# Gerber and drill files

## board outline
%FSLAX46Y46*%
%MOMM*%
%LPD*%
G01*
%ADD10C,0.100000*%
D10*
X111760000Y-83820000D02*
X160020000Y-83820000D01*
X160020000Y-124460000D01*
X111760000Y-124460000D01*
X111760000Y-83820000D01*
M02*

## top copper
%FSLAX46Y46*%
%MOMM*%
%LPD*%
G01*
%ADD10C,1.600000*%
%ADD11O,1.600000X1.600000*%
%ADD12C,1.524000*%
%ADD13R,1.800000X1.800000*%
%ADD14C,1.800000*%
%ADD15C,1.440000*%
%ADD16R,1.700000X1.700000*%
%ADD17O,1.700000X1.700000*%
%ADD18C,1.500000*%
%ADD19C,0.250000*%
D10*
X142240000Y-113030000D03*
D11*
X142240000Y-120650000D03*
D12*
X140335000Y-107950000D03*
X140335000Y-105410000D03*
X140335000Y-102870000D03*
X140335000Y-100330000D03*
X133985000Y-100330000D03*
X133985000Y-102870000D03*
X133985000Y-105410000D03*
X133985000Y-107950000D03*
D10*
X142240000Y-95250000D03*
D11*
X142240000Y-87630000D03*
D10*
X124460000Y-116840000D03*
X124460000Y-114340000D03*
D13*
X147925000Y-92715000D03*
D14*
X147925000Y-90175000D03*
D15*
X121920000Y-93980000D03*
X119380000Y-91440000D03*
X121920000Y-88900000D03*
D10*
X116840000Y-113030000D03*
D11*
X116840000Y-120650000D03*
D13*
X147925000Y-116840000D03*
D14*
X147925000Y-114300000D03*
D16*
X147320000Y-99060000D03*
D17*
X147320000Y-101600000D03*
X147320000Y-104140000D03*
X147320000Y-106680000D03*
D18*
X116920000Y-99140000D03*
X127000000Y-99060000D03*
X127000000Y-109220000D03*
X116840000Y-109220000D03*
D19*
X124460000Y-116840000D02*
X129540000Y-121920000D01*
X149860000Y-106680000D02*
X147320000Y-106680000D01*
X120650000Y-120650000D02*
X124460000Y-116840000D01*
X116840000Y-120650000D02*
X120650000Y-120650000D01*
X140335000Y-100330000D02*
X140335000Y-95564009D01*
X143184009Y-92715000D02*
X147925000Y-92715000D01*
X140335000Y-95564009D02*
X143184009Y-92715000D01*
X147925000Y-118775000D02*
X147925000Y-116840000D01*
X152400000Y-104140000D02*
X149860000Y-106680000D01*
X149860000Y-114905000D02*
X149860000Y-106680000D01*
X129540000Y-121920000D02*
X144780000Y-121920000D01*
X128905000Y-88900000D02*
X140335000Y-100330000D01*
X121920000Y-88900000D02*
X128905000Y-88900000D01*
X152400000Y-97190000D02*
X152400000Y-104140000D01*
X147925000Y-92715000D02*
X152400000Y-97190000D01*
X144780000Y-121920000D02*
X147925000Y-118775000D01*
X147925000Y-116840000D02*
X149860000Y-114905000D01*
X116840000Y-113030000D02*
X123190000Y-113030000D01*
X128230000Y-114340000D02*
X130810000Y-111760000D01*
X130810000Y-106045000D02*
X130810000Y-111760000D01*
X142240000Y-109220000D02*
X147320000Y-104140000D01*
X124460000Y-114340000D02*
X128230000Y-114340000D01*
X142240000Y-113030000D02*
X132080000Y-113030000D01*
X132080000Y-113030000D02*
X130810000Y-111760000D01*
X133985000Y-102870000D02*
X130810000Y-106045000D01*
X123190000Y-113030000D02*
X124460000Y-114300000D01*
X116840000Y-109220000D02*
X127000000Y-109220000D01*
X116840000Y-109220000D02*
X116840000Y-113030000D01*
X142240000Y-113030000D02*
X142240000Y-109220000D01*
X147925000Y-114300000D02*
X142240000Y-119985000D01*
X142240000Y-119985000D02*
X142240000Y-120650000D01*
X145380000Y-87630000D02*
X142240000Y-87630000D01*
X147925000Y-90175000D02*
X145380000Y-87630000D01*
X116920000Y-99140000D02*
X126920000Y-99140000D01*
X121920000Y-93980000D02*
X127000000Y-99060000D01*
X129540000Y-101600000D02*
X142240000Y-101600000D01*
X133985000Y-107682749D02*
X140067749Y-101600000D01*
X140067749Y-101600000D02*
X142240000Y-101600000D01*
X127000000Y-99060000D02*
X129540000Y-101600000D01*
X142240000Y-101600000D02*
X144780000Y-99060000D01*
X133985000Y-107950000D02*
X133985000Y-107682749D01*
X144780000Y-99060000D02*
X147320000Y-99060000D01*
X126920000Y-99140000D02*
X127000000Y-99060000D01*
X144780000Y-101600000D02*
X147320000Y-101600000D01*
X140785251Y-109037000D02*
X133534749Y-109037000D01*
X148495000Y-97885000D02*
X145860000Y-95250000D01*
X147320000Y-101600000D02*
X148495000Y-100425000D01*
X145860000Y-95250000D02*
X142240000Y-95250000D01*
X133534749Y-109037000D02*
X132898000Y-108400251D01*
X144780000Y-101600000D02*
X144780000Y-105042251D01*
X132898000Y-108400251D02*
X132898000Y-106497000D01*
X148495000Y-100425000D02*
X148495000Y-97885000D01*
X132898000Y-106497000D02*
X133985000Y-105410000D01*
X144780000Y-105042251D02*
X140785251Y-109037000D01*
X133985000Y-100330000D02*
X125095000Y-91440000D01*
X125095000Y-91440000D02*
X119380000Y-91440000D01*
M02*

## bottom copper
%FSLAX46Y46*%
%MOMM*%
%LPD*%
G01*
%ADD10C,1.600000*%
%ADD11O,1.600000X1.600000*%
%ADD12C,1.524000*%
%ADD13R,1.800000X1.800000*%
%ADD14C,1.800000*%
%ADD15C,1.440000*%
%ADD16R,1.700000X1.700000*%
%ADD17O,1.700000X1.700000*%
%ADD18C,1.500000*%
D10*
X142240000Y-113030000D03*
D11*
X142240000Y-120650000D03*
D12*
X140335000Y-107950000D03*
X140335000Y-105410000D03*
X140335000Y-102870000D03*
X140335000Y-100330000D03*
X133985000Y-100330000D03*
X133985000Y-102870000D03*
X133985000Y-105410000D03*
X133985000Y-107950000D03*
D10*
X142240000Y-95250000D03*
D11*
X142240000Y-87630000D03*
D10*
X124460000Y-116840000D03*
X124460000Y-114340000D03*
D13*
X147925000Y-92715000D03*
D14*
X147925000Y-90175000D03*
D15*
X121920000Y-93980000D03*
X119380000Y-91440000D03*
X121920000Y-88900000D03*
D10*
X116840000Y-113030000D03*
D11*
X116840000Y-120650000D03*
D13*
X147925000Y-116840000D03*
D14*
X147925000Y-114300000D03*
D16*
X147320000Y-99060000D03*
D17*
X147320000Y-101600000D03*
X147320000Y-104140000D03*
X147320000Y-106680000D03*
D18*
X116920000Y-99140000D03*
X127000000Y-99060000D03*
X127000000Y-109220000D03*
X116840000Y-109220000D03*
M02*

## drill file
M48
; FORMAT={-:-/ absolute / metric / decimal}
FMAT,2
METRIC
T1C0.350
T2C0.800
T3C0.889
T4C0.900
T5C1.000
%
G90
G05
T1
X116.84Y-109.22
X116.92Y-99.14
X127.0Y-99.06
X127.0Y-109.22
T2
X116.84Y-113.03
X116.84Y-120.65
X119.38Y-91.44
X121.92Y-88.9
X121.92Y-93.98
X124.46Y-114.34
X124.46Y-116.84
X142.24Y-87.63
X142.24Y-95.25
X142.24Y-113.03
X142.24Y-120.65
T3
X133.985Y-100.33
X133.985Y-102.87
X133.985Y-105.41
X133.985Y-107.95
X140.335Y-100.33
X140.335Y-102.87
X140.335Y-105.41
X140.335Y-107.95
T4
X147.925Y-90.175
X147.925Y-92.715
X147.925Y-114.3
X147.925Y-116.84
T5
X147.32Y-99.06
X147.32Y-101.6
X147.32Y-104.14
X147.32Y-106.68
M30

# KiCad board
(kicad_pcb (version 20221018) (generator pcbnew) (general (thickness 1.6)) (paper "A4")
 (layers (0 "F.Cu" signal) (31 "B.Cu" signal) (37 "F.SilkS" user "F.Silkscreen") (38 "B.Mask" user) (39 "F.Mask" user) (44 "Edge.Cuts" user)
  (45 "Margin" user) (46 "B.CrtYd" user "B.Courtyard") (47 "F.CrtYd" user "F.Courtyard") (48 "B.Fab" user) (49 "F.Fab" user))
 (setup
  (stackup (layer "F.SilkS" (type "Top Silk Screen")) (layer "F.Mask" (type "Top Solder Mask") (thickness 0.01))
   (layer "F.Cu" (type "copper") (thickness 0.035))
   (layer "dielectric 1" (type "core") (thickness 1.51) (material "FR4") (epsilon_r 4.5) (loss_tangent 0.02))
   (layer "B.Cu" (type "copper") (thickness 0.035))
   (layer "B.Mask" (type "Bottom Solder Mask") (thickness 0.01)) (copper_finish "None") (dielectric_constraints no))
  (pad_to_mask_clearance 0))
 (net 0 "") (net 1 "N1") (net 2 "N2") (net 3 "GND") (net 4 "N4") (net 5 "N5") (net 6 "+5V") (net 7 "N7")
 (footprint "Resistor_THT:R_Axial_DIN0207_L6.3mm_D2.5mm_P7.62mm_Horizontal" (layer "F.Cu") (at 142.24 113.03 -90)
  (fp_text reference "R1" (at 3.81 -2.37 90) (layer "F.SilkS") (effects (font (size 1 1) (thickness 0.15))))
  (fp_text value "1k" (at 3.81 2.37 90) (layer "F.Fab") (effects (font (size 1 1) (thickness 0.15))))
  (pad "1" thru_hole circle (at 0 0 270) (size 1.6 1.6) (drill 0.8) (layers "*.Cu" "*.Mask") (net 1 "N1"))
  (pad "2" thru_hole oval (at 7.62 0 270) (size 1.6 1.6) (drill 0.8) (layers "*.Cu" "*.Mask") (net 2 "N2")))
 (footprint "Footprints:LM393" (layer "F.Cu") (at 137.16 104.14 90)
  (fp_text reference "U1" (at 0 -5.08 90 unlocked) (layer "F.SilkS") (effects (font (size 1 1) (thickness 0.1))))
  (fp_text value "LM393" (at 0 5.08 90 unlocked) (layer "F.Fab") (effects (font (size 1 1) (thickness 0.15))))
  (pad "1" thru_hole circle (at -3.81 3.175 90) (size 1.524 1.524) (drill 0.889) (layers "*.Cu" "*.Mask"))
  (pad "2" thru_hole circle (at -1.27 3.175 90) (size 1.524 1.524) (drill 0.889) (layers "*.Cu" "*.Mask"))
  (pad "3" thru_hole circle (at 1.27 3.175 90) (size 1.524 1.524) (drill 0.889) (layers "*.Cu" "*.Mask"))
  (pad "4" thru_hole circle (at 3.81 3.175 90) (size 1.524 1.524) (drill 0.889) (layers "*.Cu" "*.Mask") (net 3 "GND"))
  (pad "5" thru_hole circle (at 3.81 -3.175 90) (size 1.524 1.524) (drill 0.889) (layers "*.Cu" "*.Mask") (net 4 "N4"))
  (pad "6" thru_hole circle (at 1.27 -3.175 90) (size 1.524 1.524) (drill 0.889) (layers "*.Cu" "*.Mask") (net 1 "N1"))
  (pad "7" thru_hole circle (at -1.27 -3.175 90) (size 1.524 1.524) (drill 0.889) (layers "*.Cu" "*.Mask") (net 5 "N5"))
  (pad "8" thru_hole circle (at -3.81 -3.175 90) (size 1.524 1.524) (drill 0.889) (layers "*.Cu" "*.Mask") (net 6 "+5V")))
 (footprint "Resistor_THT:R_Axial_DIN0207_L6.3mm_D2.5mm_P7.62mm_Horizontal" (layer "F.Cu") (at 142.24 95.25 90)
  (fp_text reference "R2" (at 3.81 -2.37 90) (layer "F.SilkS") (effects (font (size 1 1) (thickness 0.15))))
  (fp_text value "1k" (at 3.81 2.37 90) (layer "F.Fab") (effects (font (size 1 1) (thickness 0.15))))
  (pad "1" thru_hole circle (at 0 0 90) (size 1.6 1.6) (drill 0.8) (layers "*.Cu" "*.Mask") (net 5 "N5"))
  (pad "2" thru_hole oval (at 7.62 0 90) (size 1.6 1.6) (drill 0.8) (layers "*.Cu" "*.Mask") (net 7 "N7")))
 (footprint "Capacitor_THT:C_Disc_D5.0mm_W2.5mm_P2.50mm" (layer "F.Cu") (at 124.46 116.84 90)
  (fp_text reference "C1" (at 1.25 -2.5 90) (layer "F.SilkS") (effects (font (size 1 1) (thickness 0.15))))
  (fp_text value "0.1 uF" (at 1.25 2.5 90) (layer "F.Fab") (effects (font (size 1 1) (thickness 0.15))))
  (pad "1" thru_hole circle (at 0 0 90) (size 1.6 1.6) (drill 0.8) (layers "*.Cu" "*.Mask") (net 3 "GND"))
  (pad "2" thru_hole circle (at 2.5 0 90) (size 1.6 1.6) (drill 0.8) (layers "*.Cu" "*.Mask") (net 1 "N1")))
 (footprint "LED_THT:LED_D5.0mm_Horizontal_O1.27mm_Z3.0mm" (layer "F.Cu") (at 147.925 92.715 90)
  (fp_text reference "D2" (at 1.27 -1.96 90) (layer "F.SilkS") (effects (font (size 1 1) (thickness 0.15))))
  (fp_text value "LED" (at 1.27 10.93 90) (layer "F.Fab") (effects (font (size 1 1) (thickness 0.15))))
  (pad "1" thru_hole rect (at 0 0 90) (size 1.8 1.8) (drill 0.9) (layers "*.Cu" "*.Mask") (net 3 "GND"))
  (pad "2" thru_hole circle (at 2.54 0 90) (size 1.8 1.8) (drill 0.9) (layers "*.Cu" "*.Mask") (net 7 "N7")))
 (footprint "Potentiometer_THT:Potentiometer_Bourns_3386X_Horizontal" (layer "F.Cu") (at 121.92 93.98 180)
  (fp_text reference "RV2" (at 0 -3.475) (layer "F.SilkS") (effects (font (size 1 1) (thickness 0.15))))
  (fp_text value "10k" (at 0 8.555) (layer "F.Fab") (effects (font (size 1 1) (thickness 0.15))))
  (pad "1" thru_hole circle (at 0 0 180) (size 1.44 1.44) (drill 0.8) (layers "*.Cu" "*.Mask") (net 6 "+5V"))
  (pad "2" thru_hole circle (at 2.54 2.54 180) (size 1.44 1.44) (drill 0.8) (layers "*.Cu" "*.Mask") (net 4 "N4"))
  (pad "3" thru_hole circle (at 0 5.08 180) (size 1.44 1.44) (drill 0.8) (layers "*.Cu" "*.Mask") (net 3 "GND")))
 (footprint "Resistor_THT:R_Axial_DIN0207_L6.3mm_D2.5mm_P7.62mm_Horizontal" (layer "F.Cu") (at 116.84 113.03 -90)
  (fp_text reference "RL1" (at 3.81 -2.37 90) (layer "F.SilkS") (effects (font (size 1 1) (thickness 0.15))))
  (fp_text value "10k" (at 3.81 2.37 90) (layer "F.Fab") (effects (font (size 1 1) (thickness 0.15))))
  (pad "1" thru_hole circle (at 0 0 270) (size 1.6 1.6) (drill 0.8) (layers "*.Cu" "*.Mask") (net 1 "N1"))
  (pad "2" thru_hole oval (at 7.62 0 270) (size 1.6 1.6) (drill 0.8) (layers "*.Cu" "*.Mask") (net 3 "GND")))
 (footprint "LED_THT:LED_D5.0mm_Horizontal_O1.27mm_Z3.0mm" (layer "F.Cu") (at 147.925 116.84 90)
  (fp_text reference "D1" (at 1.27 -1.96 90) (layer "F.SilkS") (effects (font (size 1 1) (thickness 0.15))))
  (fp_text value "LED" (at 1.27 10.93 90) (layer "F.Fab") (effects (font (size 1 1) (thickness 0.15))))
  (pad "1" thru_hole rect (at 0 0 90) (size 1.8 1.8) (drill 0.9) (layers "*.Cu" "*.Mask") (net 3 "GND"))
  (pad "2" thru_hole circle (at 2.54 0 90) (size 1.8 1.8) (drill 0.9) (layers "*.Cu" "*.Mask") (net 2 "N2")))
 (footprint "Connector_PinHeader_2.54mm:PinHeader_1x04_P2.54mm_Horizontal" (layer "F.Cu") (at 147.32 99.06)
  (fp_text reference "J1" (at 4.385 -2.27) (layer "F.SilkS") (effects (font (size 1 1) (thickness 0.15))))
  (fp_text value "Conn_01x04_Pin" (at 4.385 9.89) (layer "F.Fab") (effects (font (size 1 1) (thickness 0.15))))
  (pad "1" thru_hole rect (at 0 0) (size 1.7 1.7) (drill 1) (layers "*.Cu" "*.Mask") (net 6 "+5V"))
  (pad "2" thru_hole oval (at 0 2.54) (size 1.7 1.7) (drill 1) (layers "*.Cu" "*.Mask") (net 5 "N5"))
  (pad "3" thru_hole oval (at 0 5.08) (size 1.7 1.7) (drill 1) (layers "*.Cu" "*.Mask") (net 1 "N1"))
  (pad "4" thru_hole oval (at 0 7.62) (size 1.7 1.7) (drill 1) (layers "*.Cu" "*.Mask") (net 3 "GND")))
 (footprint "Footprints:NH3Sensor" (layer "F.Cu") (at 121.92 104.14)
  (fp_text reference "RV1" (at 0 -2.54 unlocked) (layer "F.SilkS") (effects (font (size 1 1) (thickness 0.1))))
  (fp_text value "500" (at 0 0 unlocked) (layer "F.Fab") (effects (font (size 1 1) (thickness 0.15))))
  (pad "1" thru_hole circle (at -5 -5) (size 1.5 1.5) (drill 0.35) (layers "*.Cu" "*.Mask") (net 6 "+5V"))
  (pad "2" thru_hole circle (at 5.08 -5.08) (size 1.5 1.5) (drill 0.35) (layers "*.Cu" "*.Mask") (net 6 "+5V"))
  (pad "3" thru_hole circle (at 5.08 5.08) (size 1.5 1.5) (drill 0.35) (layers "*.Cu" "*.Mask") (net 1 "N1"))
  (pad "4" thru_hole circle (at -5.08 5.08) (size 1.5 1.5) (drill 0.35) (layers "*.Cu" "*.Mask") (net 1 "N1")))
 (gr_rect (start 111.76 83.82) (end 160.02 124.46) (stroke (width 0.1) (type default)) (fill none) (layer "Edge.Cuts"))
 (segment (start 124.46 116.84) (end 129.54 121.92) (width 0.25) (layer "F.Cu") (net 3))
 (segment (start 149.86 106.68) (end 147.32 106.68) (width 0.25) (layer "F.Cu") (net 3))
 (segment (start 120.65 120.65) (end 124.46 116.84) (width 0.25) (layer "F.Cu") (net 3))
 (segment (start 116.84 120.65) (end 120.65 120.65) (width 0.25) (layer "F.Cu") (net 3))
 (segment (start 140.335 100.33) (end 140.335 95.564009) (width 0.25) (layer "F.Cu") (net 3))
 (segment (start 143.184009 92.715) (end 147.925 92.715) (width 0.25) (layer "F.Cu") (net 3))
 (segment (start 140.335 95.564009) (end 143.184009 92.715) (width 0.25) (layer "F.Cu") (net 3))
 (segment (start 147.925 118.775) (end 147.925 116.84) (width 0.25) (layer "F.Cu") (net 3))
 (segment (start 152.4 104.14) (end 149.86 106.68) (width 0.25) (layer "F.Cu") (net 3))
 (segment (start 149.86 114.905) (end 149.86 106.68) (width 0.25) (layer "F.Cu") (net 3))
 (segment (start 129.54 121.92) (end 144.78 121.92) (width 0.25) (layer "F.Cu") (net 3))
 (segment (start 128.905 88.9) (end 140.335 100.33) (width 0.25) (layer "F.Cu") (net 3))
 (segment (start 121.92 88.9) (end 128.905 88.9) (width 0.25) (layer "F.Cu") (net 3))
 (segment (start 152.4 97.19) (end 152.4 104.14) (width 0.25) (layer "F.Cu") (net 3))
 (segment (start 147.925 92.715) (end 152.4 97.19) (width 0.25) (layer "F.Cu") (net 3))
 (segment (start 144.78 121.92) (end 147.925 118.775) (width 0.25) (layer "F.Cu") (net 3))
 (segment (start 147.925 116.84) (end 149.86 114.905) (width 0.25) (layer "F.Cu") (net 3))
 (segment (start 116.84 113.03) (end 123.19 113.03) (width 0.25) (layer "F.Cu") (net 1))
 (segment (start 128.23 114.34) (end 130.81 111.76) (width 0.25) (layer "F.Cu") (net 1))
 (segment (start 130.81 106.045) (end 130.81 111.76) (width 0.25) (layer "F.Cu") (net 1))
 (segment (start 142.24 109.22) (end 147.32 104.14) (width 0.25) (layer "F.Cu") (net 1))
 (segment (start 124.46 114.34) (end 128.23 114.34) (width 0.25) (layer "F.Cu") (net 1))
 (segment (start 142.24 113.03) (end 132.08 113.03) (width 0.25) (layer "F.Cu") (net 1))
 (segment (start 132.08 113.03) (end 130.81 111.76) (width 0.25) (layer "F.Cu") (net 1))
 (segment (start 133.985 102.87) (end 130.81 106.045) (width 0.25) (layer "F.Cu") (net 1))
 (segment (start 123.19 113.03) (end 124.46 114.3) (width 0.25) (layer "F.Cu") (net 1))
 (segment (start 116.84 109.22) (end 127 109.22) (width 0.25) (layer "F.Cu") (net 1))
 (segment (start 116.84 109.22) (end 116.84 113.03) (width 0.25) (layer "F.Cu") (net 1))
 (segment (start 142.24 113.03) (end 142.24 109.22) (width 0.25) (layer "F.Cu") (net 1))
 (segment (start 147.925 114.3) (end 142.24 119.985) (width 0.25) (layer "F.Cu") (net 2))
 (segment (start 142.24 119.985) (end 142.24 120.65) (width 0.25) (layer "F.Cu") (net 2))
 (segment (start 145.38 87.63) (end 142.24 87.63) (width 0.25) (layer "F.Cu") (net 7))
 (segment (start 147.925 90.175) (end 145.38 87.63) (width 0.25) (layer "F.Cu") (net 7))
 (segment (start 116.92 99.14) (end 126.92 99.14) (width 0.25) (layer "F.Cu") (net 6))
 (segment (start 121.92 93.98) (end 127 99.06) (width 0.25) (layer "F.Cu") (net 6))
 (segment (start 129.54 101.6) (end 142.24 101.6) (width 0.25) (layer "F.Cu") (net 6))
 (segment (start 133.985 107.682749) (end 140.067749 101.6) (width 0.25) (layer "F.Cu") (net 6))
 (segment (start 140.067749 101.6) (end 142.24 101.6) (width 0.25) (layer "F.Cu") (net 6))
 (segment (start 127 99.06) (end 129.54 101.6) (width 0.25) (layer "F.Cu") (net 6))
 (segment (start 142.24 101.6) (end 144.78 99.06) (width 0.25) (layer "F.Cu") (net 6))
 (segment (start 133.985 107.95) (end 133.985 107.682749) (width 0.25) (layer "F.Cu") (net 6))
 (segment (start 144.78 99.06) (end 147.32 99.06) (width 0.25) (layer "F.Cu") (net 6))
 (segment (start 126.92 99.14) (end 127 99.06) (width 0.25) (layer "F.Cu") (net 6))
 (segment (start 144.78 101.6) (end 147.32 101.6) (width 0.25) (layer "F.Cu") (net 5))
 (segment (start 140.785251 109.037) (end 133.534749 109.037) (width 0.25) (layer "F.Cu") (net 5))
 (segment (start 148.495 97.885) (end 145.86 95.25) (width 0.25) (layer "F.Cu") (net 5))
 (segment (start 147.32 101.6) (end 148.495 100.425) (width 0.25) (layer "F.Cu") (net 5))
 (segment (start 145.86 95.25) (end 142.24 95.25) (width 0.25) (layer "F.Cu") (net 5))
 (segment (start 133.534749 109.037) (end 132.898 108.400251) (width 0.25) (layer "F.Cu") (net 5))
 (segment (start 144.78 101.6) (end 144.78 105.042251) (width 0.25) (layer "F.Cu") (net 5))
 (segment (start 132.898 108.400251) (end 132.898 106.497) (width 0.25) (layer "F.Cu") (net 5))
 (segment (start 148.495 100.425) (end 148.495 97.885) (width 0.25) (layer "F.Cu") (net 5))
 (segment (start 132.898 106.497) (end 133.985 105.41) (width 0.25) (layer "F.Cu") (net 5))
 (segment (start 144.78 105.042251) (end 140.785251 109.037) (width 0.25) (layer "F.Cu") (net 5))
 (segment (start 133.985 100.33) (end 125.095 91.44) (width 0.25) (layer "F.Cu") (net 4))
 (segment (start 125.095 91.44) (end 119.38 91.44) (width 0.25) (layer "F.Cu") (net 4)))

